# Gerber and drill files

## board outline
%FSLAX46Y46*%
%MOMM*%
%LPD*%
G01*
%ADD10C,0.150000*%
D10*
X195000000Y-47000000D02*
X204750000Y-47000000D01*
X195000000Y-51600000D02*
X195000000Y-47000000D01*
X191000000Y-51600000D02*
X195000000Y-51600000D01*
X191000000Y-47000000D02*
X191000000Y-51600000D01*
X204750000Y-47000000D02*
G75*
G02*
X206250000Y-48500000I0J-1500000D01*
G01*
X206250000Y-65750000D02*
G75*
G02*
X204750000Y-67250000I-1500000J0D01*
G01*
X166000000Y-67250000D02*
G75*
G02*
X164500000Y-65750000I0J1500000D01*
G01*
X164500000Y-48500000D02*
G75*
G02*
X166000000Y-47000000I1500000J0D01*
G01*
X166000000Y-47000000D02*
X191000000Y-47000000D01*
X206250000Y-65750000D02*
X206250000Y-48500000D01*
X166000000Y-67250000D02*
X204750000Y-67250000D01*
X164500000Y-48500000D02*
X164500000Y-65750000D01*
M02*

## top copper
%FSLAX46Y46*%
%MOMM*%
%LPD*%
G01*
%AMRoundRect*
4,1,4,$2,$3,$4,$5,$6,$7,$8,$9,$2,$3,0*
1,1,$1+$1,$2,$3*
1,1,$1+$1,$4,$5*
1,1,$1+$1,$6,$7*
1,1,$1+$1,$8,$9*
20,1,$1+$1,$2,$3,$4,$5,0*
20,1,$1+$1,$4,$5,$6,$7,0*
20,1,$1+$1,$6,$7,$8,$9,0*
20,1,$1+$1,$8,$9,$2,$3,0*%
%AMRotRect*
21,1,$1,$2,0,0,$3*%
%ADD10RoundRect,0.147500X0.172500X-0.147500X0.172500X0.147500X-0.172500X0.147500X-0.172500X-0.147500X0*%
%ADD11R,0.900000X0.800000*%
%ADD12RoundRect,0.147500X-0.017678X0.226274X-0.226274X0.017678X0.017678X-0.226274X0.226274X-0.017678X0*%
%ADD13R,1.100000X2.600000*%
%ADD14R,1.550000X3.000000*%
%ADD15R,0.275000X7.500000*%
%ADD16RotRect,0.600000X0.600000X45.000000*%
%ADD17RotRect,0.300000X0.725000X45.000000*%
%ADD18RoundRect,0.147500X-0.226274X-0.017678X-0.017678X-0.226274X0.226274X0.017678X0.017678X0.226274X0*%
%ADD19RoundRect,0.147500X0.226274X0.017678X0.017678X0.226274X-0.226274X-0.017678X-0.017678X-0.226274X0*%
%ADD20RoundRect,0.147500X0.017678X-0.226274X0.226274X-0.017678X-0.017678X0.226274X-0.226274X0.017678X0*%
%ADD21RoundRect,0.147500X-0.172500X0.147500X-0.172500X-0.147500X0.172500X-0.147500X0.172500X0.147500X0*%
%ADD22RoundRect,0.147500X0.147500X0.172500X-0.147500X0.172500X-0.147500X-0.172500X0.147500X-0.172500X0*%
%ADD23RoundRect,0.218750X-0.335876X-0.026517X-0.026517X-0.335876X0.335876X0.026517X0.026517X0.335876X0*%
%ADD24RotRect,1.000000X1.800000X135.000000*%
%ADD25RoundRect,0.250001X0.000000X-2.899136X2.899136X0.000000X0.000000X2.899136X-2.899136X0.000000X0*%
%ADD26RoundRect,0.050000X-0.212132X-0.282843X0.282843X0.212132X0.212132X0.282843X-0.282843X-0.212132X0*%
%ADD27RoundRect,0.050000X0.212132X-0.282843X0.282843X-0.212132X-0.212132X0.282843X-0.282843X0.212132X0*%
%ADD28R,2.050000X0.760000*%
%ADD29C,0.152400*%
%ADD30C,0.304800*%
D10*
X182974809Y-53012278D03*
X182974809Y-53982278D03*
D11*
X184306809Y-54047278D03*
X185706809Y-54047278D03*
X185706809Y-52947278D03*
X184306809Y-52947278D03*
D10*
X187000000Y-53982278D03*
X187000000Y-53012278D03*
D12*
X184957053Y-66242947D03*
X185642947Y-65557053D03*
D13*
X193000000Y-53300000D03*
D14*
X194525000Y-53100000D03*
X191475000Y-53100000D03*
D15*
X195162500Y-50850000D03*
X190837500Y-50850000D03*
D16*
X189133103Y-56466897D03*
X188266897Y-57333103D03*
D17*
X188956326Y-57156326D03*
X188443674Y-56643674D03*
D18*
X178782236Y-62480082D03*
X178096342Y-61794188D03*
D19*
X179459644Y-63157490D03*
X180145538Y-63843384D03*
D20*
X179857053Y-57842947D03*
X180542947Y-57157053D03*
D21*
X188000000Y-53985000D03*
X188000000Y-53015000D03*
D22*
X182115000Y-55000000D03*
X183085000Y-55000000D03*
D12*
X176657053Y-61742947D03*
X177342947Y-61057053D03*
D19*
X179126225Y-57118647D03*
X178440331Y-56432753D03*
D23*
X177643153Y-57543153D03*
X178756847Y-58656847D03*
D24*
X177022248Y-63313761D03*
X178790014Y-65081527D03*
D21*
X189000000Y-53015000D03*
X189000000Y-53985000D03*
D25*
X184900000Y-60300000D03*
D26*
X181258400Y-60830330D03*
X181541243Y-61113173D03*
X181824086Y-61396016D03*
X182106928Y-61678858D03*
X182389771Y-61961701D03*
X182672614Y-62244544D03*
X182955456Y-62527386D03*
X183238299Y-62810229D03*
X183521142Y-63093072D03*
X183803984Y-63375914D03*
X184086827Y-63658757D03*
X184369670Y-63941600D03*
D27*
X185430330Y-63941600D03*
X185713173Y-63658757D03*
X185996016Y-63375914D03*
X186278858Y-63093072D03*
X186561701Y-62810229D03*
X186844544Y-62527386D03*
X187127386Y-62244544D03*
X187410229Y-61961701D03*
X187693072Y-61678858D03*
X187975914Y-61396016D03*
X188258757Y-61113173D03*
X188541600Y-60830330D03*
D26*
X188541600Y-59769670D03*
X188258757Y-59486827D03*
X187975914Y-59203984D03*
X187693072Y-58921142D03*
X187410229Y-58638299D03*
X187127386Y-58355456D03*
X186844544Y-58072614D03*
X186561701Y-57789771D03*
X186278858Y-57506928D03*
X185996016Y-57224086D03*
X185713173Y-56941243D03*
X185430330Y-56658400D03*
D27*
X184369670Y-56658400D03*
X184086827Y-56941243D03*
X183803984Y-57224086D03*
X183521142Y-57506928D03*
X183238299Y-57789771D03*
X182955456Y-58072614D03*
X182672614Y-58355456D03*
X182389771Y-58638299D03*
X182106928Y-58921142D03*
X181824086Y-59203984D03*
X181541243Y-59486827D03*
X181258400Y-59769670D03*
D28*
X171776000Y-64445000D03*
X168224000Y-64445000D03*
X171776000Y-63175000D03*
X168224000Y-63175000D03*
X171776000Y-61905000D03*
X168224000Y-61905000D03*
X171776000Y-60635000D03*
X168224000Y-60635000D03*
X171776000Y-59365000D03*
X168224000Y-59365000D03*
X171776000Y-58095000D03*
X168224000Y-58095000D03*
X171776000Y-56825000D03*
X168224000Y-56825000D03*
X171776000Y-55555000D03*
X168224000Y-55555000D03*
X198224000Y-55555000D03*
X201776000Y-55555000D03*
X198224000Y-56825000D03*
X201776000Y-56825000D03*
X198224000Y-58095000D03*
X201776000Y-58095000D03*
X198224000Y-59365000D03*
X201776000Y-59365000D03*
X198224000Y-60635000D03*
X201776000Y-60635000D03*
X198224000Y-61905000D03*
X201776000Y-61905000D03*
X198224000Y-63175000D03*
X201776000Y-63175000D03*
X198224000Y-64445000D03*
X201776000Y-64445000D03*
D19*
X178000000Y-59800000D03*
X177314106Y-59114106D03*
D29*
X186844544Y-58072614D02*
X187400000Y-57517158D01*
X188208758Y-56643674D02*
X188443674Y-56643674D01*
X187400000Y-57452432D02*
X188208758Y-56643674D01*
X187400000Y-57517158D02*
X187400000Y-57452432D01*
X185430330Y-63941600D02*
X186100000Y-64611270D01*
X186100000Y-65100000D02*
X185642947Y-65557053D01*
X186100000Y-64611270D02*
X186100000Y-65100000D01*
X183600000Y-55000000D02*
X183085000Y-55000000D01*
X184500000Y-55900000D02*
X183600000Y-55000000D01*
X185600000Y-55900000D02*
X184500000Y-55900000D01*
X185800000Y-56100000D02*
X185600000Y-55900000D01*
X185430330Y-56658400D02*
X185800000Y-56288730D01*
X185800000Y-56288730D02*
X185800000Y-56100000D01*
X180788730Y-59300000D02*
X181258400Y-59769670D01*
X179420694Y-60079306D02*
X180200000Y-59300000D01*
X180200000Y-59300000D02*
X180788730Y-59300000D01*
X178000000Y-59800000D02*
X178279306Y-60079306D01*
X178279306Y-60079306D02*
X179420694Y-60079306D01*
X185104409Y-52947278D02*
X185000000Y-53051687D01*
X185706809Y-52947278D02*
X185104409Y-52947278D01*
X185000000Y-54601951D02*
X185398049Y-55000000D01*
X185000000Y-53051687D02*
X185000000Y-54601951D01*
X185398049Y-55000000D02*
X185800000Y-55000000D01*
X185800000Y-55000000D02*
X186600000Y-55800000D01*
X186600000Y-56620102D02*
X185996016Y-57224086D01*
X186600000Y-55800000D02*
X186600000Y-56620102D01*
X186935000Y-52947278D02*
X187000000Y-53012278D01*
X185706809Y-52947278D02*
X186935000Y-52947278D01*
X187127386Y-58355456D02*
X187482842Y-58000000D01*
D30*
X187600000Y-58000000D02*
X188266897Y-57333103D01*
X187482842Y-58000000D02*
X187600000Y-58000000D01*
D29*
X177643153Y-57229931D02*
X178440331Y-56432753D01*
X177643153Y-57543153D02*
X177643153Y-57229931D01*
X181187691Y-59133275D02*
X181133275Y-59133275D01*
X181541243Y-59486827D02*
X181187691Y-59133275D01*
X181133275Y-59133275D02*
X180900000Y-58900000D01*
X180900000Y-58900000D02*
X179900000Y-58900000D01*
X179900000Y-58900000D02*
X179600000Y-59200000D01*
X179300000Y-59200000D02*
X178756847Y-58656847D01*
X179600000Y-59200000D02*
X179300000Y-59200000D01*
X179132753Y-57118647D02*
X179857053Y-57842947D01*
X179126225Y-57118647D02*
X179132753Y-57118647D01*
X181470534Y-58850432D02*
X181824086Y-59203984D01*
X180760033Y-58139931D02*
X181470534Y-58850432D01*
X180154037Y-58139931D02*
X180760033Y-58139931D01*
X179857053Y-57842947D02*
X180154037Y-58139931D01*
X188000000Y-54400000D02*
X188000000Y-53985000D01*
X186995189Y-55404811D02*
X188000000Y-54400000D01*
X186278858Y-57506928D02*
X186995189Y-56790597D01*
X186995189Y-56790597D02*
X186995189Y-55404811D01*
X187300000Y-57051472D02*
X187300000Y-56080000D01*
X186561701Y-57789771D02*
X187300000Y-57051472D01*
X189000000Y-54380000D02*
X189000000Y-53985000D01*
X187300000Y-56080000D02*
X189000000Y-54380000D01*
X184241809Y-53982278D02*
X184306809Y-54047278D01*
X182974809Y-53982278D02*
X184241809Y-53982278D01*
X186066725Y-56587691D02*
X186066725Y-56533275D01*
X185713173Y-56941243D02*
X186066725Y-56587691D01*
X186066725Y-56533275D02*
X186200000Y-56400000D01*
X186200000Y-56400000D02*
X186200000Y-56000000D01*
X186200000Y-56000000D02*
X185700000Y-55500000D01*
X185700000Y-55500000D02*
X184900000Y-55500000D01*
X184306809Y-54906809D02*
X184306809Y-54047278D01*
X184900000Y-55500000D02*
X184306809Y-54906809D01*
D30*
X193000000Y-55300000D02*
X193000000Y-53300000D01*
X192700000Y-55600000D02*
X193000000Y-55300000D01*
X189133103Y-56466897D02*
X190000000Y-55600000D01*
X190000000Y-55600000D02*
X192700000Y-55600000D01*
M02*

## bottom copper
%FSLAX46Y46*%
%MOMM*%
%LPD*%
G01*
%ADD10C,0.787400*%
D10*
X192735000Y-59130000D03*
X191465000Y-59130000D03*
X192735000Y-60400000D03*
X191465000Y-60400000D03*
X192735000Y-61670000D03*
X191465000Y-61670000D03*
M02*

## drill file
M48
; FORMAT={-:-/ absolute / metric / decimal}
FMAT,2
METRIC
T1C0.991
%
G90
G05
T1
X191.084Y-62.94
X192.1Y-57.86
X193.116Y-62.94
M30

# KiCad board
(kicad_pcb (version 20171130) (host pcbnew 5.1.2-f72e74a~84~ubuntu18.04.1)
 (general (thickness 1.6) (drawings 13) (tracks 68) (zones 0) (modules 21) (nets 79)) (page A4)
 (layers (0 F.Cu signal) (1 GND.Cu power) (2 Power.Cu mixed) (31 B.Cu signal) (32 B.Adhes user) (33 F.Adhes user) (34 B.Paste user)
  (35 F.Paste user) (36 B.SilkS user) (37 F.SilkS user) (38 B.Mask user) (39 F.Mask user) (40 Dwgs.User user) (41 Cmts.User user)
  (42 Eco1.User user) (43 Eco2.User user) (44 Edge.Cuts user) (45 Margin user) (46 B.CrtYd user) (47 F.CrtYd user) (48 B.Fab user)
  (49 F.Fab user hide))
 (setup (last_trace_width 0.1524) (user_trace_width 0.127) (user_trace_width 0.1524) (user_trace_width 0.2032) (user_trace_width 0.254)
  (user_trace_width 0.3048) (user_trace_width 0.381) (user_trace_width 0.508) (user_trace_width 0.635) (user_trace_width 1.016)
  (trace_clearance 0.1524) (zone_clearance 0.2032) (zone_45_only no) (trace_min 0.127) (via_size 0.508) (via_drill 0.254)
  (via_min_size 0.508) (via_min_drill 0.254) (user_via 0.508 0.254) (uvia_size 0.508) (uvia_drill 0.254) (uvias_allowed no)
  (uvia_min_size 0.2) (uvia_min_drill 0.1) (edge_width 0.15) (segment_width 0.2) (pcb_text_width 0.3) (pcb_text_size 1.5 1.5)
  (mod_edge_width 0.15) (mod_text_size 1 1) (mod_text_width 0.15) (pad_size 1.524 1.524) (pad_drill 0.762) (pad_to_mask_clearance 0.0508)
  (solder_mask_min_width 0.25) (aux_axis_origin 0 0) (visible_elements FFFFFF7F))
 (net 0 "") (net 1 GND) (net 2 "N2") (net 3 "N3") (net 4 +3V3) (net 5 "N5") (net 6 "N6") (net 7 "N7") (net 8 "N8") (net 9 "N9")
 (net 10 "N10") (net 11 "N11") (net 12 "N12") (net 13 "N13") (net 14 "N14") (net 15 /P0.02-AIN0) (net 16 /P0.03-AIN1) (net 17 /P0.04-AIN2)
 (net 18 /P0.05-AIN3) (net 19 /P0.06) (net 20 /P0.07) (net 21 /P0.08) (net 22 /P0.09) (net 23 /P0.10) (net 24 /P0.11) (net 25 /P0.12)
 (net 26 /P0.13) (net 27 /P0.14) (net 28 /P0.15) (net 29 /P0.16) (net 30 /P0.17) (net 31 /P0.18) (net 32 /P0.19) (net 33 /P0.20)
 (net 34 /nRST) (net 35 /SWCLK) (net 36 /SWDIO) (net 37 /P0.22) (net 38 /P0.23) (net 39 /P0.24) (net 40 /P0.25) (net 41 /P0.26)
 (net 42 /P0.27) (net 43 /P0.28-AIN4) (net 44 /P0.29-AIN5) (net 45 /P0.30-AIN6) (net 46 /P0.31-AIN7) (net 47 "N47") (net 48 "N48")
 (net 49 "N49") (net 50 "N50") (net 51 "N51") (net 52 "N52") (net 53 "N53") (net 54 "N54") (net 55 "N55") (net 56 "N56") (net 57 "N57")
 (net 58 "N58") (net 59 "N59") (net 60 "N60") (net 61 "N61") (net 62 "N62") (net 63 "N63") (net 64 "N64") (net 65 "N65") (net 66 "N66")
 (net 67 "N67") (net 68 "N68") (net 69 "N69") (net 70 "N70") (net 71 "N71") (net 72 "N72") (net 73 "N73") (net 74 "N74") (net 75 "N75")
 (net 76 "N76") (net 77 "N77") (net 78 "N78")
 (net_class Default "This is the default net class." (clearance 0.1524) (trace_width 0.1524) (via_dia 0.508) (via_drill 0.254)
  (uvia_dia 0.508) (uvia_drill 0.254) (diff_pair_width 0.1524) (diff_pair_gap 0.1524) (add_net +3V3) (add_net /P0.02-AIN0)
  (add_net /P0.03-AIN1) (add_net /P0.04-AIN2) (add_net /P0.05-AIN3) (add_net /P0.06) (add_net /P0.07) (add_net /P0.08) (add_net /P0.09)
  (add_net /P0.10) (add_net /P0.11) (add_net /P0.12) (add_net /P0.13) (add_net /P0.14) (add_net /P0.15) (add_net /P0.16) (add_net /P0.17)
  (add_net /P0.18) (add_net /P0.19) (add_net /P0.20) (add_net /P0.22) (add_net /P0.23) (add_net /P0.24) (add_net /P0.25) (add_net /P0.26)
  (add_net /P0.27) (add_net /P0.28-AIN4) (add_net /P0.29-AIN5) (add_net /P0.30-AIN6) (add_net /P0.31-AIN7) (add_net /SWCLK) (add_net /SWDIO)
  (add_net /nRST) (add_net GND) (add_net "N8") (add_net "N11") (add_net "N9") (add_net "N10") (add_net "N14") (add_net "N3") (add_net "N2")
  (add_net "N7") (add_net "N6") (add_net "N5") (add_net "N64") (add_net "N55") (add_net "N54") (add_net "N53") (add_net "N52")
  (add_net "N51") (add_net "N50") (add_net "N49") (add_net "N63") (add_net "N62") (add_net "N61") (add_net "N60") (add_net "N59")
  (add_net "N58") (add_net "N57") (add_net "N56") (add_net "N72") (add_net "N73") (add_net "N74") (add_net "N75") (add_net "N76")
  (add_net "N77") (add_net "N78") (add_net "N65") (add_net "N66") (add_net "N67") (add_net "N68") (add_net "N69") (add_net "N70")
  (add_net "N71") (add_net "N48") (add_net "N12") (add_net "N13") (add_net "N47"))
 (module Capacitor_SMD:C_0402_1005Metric (layer F.Cu) (at 182.974809 53.497278 90)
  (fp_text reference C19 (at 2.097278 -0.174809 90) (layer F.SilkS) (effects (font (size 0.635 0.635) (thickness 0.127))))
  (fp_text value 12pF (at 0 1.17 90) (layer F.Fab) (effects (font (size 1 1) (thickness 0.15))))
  (pad 2 smd roundrect (at 0.485 0 90) (size 0.59 0.64) (layers F.Cu F.Paste F.Mask) (roundrect_rratio 0.25) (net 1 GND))
  (pad 1 smd roundrect (at -0.485 0 90) (size 0.59 0.64) (layers F.Cu F.Paste F.Mask) (roundrect_rratio 0.25) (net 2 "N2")))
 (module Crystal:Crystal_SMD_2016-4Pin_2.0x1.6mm (layer F.Cu) (at 185.006809 53.497278)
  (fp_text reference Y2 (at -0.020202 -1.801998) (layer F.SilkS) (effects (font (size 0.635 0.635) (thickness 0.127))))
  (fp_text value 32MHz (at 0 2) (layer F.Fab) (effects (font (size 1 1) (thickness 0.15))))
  (pad 1 smd rect (at -0.7 0.55) (size 0.9 0.8) (layers F.Cu F.Paste F.Mask) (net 2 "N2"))
  (pad 2 smd rect (at 0.7 0.55) (size 0.9 0.8) (layers F.Cu F.Paste F.Mask) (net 1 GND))
  (pad 3 smd rect (at 0.7 -0.55) (size 0.9 0.8) (layers F.Cu F.Paste F.Mask) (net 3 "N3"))
  (pad 4 smd rect (at -0.7 -0.55) (size 0.9 0.8) (layers F.Cu F.Paste F.Mask) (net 1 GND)))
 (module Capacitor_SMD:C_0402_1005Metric (layer F.Cu) (at 187 53.497278 90)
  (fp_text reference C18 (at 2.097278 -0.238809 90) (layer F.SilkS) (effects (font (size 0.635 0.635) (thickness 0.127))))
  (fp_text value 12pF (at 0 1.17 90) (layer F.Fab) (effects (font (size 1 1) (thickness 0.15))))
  (pad 1 smd roundrect (at -0.485 0 90) (size 0.59 0.64) (layers F.Cu F.Paste F.Mask) (roundrect_rratio 0.25) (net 1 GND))
  (pad 2 smd roundrect (at 0.485 0 90) (size 0.59 0.64) (layers F.Cu F.Paste F.Mask) (roundrect_rratio 0.25) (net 3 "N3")))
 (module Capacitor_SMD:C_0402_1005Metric (layer F.Cu) (at 185.3 65.9 225)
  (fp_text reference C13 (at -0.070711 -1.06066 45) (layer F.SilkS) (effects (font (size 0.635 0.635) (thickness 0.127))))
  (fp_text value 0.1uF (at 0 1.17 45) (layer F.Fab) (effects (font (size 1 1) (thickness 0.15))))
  (pad 2 smd roundrect (at 0.485 0 225) (size 0.59 0.64) (layers F.Cu F.Paste F.Mask) (roundrect_rratio 0.25) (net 1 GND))
  (pad 1 smd roundrect (at -0.485 0 225) (size 0.59 0.64) (layers F.Cu F.Paste F.Mask) (roundrect_rratio 0.25) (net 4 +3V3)))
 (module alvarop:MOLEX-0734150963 (layer F.Cu) (at 193 54.6 270)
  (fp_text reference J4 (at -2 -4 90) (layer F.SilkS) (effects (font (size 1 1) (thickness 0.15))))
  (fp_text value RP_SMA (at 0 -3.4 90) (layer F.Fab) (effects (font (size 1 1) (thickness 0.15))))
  (pad 1 smd rect (at -1.3 0 270) (size 2.6 1.1) (layers F.Cu F.Paste F.Mask) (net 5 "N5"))
  (pad 2 smd rect (at -1.5 -1.525 270) (size 3 1.55) (layers F.Cu F.Paste F.Mask) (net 1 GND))
  (pad 2 smd rect (at -1.5 1.525 270) (size 3 1.55) (layers F.Cu F.Paste F.Mask) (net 1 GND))
  (pad 2 smd rect (at -3.75 -2.1625 270) (size 7.5 0.275) (layers F.Cu F.Paste F.Mask) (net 1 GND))
  (pad 2 smd rect (at -3.75 2.1625 270) (size 7.5 0.275) (layers F.Cu F.Paste F.Mask) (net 1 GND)))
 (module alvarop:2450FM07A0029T (layer F.Cu) (at 188.7 56.9 45)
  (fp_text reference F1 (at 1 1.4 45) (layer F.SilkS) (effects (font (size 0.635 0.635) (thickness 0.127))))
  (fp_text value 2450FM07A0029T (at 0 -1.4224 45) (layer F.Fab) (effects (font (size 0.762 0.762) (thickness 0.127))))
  (pad 3 smd rect (at 0.6125 0 45) (size 0.6 0.6) (layers F.Cu F.Paste F.Mask) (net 5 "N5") (solder_paste_margin -0.0508))
  (pad 1 smd rect (at -0.6125 0 45) (size 0.6 0.6) (layers F.Cu F.Paste F.Mask) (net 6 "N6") (solder_paste_margin -0.0508))
  (pad 2 smd rect (at 0 0.3625 45) (size 0.3 0.725) (layers F.Cu F.Paste F.Mask) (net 1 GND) (solder_paste_margin -0.0508))
  (pad 4 smd rect (at 0 -0.3625 45) (size 0.3 0.725) (layers F.Cu F.Paste F.Mask) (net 1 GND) (solder_paste_margin -0.0508)))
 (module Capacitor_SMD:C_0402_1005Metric (layer F.Cu) (at 178.439289 62.137135 315)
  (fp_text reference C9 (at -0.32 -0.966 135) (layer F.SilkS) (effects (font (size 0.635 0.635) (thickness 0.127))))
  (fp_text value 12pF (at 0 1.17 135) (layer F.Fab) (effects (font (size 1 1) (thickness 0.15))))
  (pad 2 smd roundrect (at 0.485 0 315) (size 0.59 0.64) (layers F.Cu F.Paste F.Mask) (roundrect_rratio 0.25) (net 1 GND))
  (pad 1 smd roundrect (at -0.485 0 315) (size 0.59 0.64) (layers F.Cu F.Paste F.Mask) (roundrect_rratio 0.25) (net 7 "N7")))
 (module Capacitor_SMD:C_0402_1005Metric (layer F.Cu) (at 179.802591 63.500437 135)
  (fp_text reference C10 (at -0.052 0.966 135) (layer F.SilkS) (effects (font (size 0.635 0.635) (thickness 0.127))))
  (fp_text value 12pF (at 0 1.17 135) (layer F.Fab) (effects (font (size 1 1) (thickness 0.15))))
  (pad 2 smd roundrect (at 0.485 0 135) (size 0.59 0.64) (layers F.Cu F.Paste F.Mask) (roundrect_rratio 0.25) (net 1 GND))
  (pad 1 smd roundrect (at -0.485 0 135) (size 0.59 0.64) (layers F.Cu F.Paste F.Mask) (roundrect_rratio 0.25) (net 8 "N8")))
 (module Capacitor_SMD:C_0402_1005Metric (layer F.Cu) (at 180.2 57.5 45)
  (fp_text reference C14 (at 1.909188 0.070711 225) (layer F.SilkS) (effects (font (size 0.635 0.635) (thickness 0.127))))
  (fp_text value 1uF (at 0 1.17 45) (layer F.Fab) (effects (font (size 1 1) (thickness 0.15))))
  (pad 1 smd roundrect (at -0.485 0 45) (size 0.59 0.64) (layers F.Cu F.Paste F.Mask) (roundrect_rratio 0.25) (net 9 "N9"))
  (pad 2 smd roundrect (at 0.485 0 45) (size 0.59 0.64) (layers F.Cu F.Paste F.Mask) (roundrect_rratio 0.25) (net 1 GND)))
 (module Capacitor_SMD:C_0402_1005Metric (layer F.Cu) (at 188 53.5 270)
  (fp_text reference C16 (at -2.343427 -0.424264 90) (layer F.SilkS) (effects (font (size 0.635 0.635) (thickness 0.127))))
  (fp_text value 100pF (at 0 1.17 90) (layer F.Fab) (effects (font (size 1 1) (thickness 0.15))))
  (pad 2 smd roundrect (at 0.485 0 270) (size 0.59 0.64) (layers F.Cu F.Paste F.Mask) (roundrect_rratio 0.25) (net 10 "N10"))
  (pad 1 smd roundrect (at -0.485 0 270) (size 0.59 0.64) (layers F.Cu F.Paste F.Mask) (roundrect_rratio 0.25) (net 1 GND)))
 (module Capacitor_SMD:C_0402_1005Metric (layer F.Cu) (at 182.6 55 180)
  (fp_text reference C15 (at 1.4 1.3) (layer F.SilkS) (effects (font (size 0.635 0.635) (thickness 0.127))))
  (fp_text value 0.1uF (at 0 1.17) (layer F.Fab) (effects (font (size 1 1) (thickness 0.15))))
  (pad 2 smd roundrect (at 0.485 0 180) (size 0.59 0.64) (layers F.Cu F.Paste F.Mask) (roundrect_rratio 0.25) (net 1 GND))
  (pad 1 smd roundrect (at -0.485 0 180) (size 0.59 0.64) (layers F.Cu F.Paste F.Mask) (roundrect_rratio 0.25) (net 4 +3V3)))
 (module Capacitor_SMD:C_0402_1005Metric (layer F.Cu) (at 177 61.4 225)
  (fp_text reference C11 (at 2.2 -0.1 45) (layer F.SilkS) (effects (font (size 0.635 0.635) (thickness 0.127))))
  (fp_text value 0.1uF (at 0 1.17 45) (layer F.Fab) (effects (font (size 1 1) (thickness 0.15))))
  (pad 2 smd roundrect (at 0.485 0 225) (size 0.59 0.64) (layers F.Cu F.Paste F.Mask) (roundrect_rratio 0.25) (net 1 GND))
  (pad 1 smd roundrect (at -0.485 0 225) (size 0.59 0.64) (layers F.Cu F.Paste F.Mask) (roundrect_rratio 0.25) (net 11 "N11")))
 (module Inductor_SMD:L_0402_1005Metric (layer F.Cu) (at 178.783278 56.7757 135)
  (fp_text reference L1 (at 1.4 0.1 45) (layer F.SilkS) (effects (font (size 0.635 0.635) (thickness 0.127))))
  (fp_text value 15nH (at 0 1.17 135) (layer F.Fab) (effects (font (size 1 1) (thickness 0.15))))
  (pad 1 smd roundrect (at -0.485 0 135) (size 0.59 0.64) (layers F.Cu F.Paste F.Mask) (roundrect_rratio 0.25) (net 9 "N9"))
  (pad 2 smd roundrect (at 0.485 0 135) (size 0.59 0.64) (layers F.Cu F.Paste F.Mask) (roundrect_rratio 0.25) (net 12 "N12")))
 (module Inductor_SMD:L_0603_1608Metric (layer F.Cu) (at 178.2 58.1 315)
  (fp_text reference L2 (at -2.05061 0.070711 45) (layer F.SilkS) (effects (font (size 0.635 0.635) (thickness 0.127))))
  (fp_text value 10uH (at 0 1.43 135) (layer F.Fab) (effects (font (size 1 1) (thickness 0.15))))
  (pad 1 smd roundrect (at -0.7875 0 315) (size 0.875 0.95) (layers F.Cu F.Paste F.Mask) (roundrect_rratio 0.25) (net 12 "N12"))
  (pad 2 smd roundrect (at 0.7875 0 315) (size 0.875 0.95) (layers F.Cu F.Paste F.Mask) (roundrect_rratio 0.25) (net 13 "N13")))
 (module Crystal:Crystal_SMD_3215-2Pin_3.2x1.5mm (layer F.Cu) (at 177.906131 64.197644 135)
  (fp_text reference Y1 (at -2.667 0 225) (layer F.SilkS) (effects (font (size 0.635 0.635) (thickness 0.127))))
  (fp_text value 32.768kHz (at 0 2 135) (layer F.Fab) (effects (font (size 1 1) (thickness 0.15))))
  (pad 1 smd rect (at 1.25 0 135) (size 1 1.8) (layers F.Cu F.Paste F.Mask) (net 7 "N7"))
  (pad 2 smd rect (at -1.25 0 135) (size 1 1.8) (layers F.Cu F.Paste F.Mask) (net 8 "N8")))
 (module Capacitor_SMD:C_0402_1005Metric (layer F.Cu) (at 189 53.5 270)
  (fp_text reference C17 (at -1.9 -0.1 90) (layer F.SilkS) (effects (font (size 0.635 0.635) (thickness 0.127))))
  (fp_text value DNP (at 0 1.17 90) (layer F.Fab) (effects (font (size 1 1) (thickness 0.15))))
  (pad 1 smd roundrect (at -0.485 0 270) (size 0.59 0.64) (layers F.Cu F.Paste F.Mask) (roundrect_rratio 0.25) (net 1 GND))
  (pad 2 smd roundrect (at 0.485 0 270) (size 0.59 0.64) (layers F.Cu F.Paste F.Mask) (roundrect_rratio 0.25) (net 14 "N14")))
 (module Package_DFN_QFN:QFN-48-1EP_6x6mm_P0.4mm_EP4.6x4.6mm (layer F.Cu) (at 184.9 60.3 45)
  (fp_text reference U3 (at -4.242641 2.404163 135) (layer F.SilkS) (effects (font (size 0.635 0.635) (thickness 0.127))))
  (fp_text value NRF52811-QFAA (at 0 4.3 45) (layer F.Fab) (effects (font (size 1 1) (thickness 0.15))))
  (pad 49 smd roundrect (at 0 0 45) (size 4.6 4.6) (layers F.Cu F.Mask) (roundrect_rratio 0.054348) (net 1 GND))
  (pad "" smd roundrect (at -1.53 -1.53 45) (size 1.24 1.24) (layers F.Paste) (roundrect_rratio 0.201613))
  (pad "" smd roundrect (at -1.53 0 45) (size 1.24 1.24) (layers F.Paste) (roundrect_rratio 0.201613))
  (pad "" smd roundrect (at -1.53 1.53 45) (size 1.24 1.24) (layers F.Paste) (roundrect_rratio 0.201613))
  (pad "" smd roundrect (at 0 -1.53 45) (size 1.24 1.24) (layers F.Paste) (roundrect_rratio 0.201613))
  (pad "" smd roundrect (at 0 0 45) (size 1.24 1.24) (layers F.Paste) (roundrect_rratio 0.201613))
  (pad "" smd roundrect (at 0 1.53 45) (size 1.24 1.24) (layers F.Paste) (roundrect_rratio 0.201613))
  (pad "" smd roundrect (at 1.53 -1.53 45) (size 1.24 1.24) (layers F.Paste) (roundrect_rratio 0.201613))
  (pad "" smd roundrect (at 1.53 0 45) (size 1.24 1.24) (layers F.Paste) (roundrect_rratio 0.201613))
  (pad "" smd roundrect (at 1.53 1.53 45) (size 1.24 1.24) (layers F.Paste) (roundrect_rratio 0.201613))
  (pad 1 smd roundrect (at -2.95 -2.2 45) (size 0.8 0.2) (layers F.Cu F.Paste F.Mask) (roundrect_rratio 0.25) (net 11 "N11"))
  (pad 2 smd roundrect (at -2.95 -1.8 45) (size 0.8 0.2) (layers F.Cu F.Paste F.Mask) (roundrect_rratio 0.25) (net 7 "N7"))
  (pad 3 smd roundrect (at -2.95 -1.4 45) (size 0.8 0.2) (layers F.Cu F.Paste F.Mask) (roundrect_rratio 0.25) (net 8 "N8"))
  (pad 4 smd roundrect (at -2.95 -1 45) (size 0.8 0.2) (layers F.Cu F.Paste F.Mask) (roundrect_rratio 0.25) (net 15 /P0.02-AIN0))
  (pad 5 smd roundrect (at -2.95 -0.6 45) (size 0.8 0.2) (layers F.Cu F.Paste F.Mask) (roundrect_rratio 0.25) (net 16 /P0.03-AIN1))
  (pad 6 smd roundrect (at -2.95 -0.2 45) (size 0.8 0.2) (layers F.Cu F.Paste F.Mask) (roundrect_rratio 0.25) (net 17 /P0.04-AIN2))
  (pad 7 smd roundrect (at -2.95 0.2 45) (size 0.8 0.2) (layers F.Cu F.Paste F.Mask) (roundrect_rratio 0.25) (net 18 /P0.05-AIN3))
  (pad 8 smd roundrect (at -2.95 0.6 45) (size 0.8 0.2) (layers F.Cu F.Paste F.Mask) (roundrect_rratio 0.25) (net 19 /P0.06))
  (pad 9 smd roundrect (at -2.95 1 45) (size 0.8 0.2) (layers F.Cu F.Paste F.Mask) (roundrect_rratio 0.25) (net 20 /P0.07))
  (pad 10 smd roundrect (at -2.95 1.4 45) (size 0.8 0.2) (layers F.Cu F.Paste F.Mask) (roundrect_rratio 0.25) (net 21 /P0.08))
  (pad 11 smd roundrect (at -2.95 1.8 45) (size 0.8 0.2) (layers F.Cu F.Paste F.Mask) (roundrect_rratio 0.25) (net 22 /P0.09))
  (pad 12 smd roundrect (at -2.95 2.2 45) (size 0.8 0.2) (layers F.Cu F.Paste F.Mask) (roundrect_rratio 0.25) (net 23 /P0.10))
  (pad 13 smd roundrect (at -2.2 2.95 45) (size 0.2 0.8) (layers F.Cu F.Paste F.Mask) (roundrect_rratio 0.25) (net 4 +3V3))
  (pad 14 smd roundrect (at -1.8 2.95 45) (size 0.2 0.8) (layers F.Cu F.Paste F.Mask) (roundrect_rratio 0.25) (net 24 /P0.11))
  (pad 15 smd roundrect (at -1.4 2.95 45) (size 0.2 0.8) (layers F.Cu F.Paste F.Mask) (roundrect_rratio 0.25) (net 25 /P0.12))
  (pad 16 smd roundrect (at -1 2.95 45) (size 0.2 0.8) (layers F.Cu F.Paste F.Mask) (roundrect_rratio 0.25) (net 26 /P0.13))
  (pad 17 smd roundrect (at -0.6 2.95 45) (size 0.2 0.8) (layers F.Cu F.Paste F.Mask) (roundrect_rratio 0.25) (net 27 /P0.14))
  (pad 18 smd roundrect (at -0.2 2.95 45) (size 0.2 0.8) (layers F.Cu F.Paste F.Mask) (roundrect_rratio 0.25) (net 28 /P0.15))
  (pad 19 smd roundrect (at 0.2 2.95 45) (size 0.2 0.8) (layers F.Cu F.Paste F.Mask) (roundrect_rratio 0.25) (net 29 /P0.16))
  (pad 20 smd roundrect (at 0.6 2.95 45) (size 0.2 0.8) (layers F.Cu F.Paste F.Mask) (roundrect_rratio 0.25) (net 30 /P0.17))
  (pad 21 smd roundrect (at 1 2.95 45) (size 0.2 0.8) (layers F.Cu F.Paste F.Mask) (roundrect_rratio 0.25) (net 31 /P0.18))
  (pad 22 smd roundrect (at 1.4 2.95 45) (size 0.2 0.8) (layers F.Cu F.Paste F.Mask) (roundrect_rratio 0.25) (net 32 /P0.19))
  (pad 23 smd roundrect (at 1.8 2.95 45) (size 0.2 0.8) (layers F.Cu F.Paste F.Mask) (roundrect_rratio 0.25) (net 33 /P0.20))
  (pad 24 smd roundrect (at 2.2 2.95 45) (size 0.2 0.8) (layers F.Cu F.Paste F.Mask) (roundrect_rratio 0.25) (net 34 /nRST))
  (pad 25 smd roundrect (at 2.95 2.2 45) (size 0.8 0.2) (layers F.Cu F.Paste F.Mask) (roundrect_rratio 0.25) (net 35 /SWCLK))
  (pad 26 smd roundrect (at 2.95 1.8 45) (size 0.8 0.2) (layers F.Cu F.Paste F.Mask) (roundrect_rratio 0.25) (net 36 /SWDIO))
  (pad 27 smd roundrect (at 2.95 1.4 45) (size 0.8 0.2) (layers F.Cu F.Paste F.Mask) (roundrect_rratio 0.25) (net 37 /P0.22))
  (pad 28 smd roundrect (at 2.95 1 45) (size 0.8 0.2) (layers F.Cu F.Paste F.Mask) (roundrect_rratio 0.25) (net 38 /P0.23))
  (pad 29 smd roundrect (at 2.95 0.6 45) (size 0.8 0.2) (layers F.Cu F.Paste F.Mask) (roundrect_rratio 0.25) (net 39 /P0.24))
  (pad 30 smd roundrect (at 2.95 0.2 45) (size 0.8 0.2) (layers F.Cu F.Paste F.Mask) (roundrect_rratio 0.25) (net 6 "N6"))
  (pad 31 smd roundrect (at 2.95 -0.2 45) (size 0.8 0.2) (layers F.Cu F.Paste F.Mask) (roundrect_rratio 0.25) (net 1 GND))
  (pad 32 smd roundrect (at 2.95 -0.6 45) (size 0.8 0.2) (layers F.Cu F.Paste F.Mask) (roundrect_rratio 0.25) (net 14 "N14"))
  (pad 33 smd roundrect (at 2.95 -1 45) (size 0.8 0.2) (layers F.Cu F.Paste F.Mask) (roundrect_rratio 0.25) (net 10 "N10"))
  (pad 34 smd roundrect (at 2.95 -1.4 45) (size 0.8 0.2) (layers F.Cu F.Paste F.Mask) (roundrect_rratio 0.25) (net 3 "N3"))
  (pad 35 smd roundrect (at 2.95 -1.8 45) (size 0.8 0.2) (layers F.Cu F.Paste F.Mask) (roundrect_rratio 0.25) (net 2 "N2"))
  (pad 36 smd roundrect (at 2.95 -2.2 45) (size 0.8 0.2) (layers F.Cu F.Paste F.Mask) (roundrect_rratio 0.25) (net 4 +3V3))
  (pad 37 smd roundrect (at 2.2 -2.95 45) (size 0.2 0.8) (layers F.Cu F.Paste F.Mask) (roundrect_rratio 0.25) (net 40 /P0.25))
  (pad 38 smd roundrect (at 1.8 -2.95 45) (size 0.2 0.8) (layers F.Cu F.Paste F.Mask) (roundrect_rratio 0.25) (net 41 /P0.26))
  (pad 39 smd roundrect (at 1.4 -2.95 45) (size 0.2 0.8) (layers F.Cu F.Paste F.Mask) (roundrect_rratio 0.25) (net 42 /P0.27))
  (pad 40 smd roundrect (at 1 -2.95 45) (size 0.2 0.8) (layers F.Cu F.Paste F.Mask) (roundrect_rratio 0.25) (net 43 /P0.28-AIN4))
  (pad 41 smd roundrect (at 0.6 -2.95 45) (size 0.2 0.8) (layers F.Cu F.Paste F.Mask) (roundrect_rratio 0.25) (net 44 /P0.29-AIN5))
  (pad 42 smd roundrect (at 0.2 -2.95 45) (size 0.2 0.8) (layers F.Cu F.Paste F.Mask) (roundrect_rratio 0.25) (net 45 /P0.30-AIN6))
  (pad 43 smd roundrect (at -0.2 -2.95 45) (size 0.2 0.8) (layers F.Cu F.Paste F.Mask) (roundrect_rratio 0.25) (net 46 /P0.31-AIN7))
  (pad 44 smd roundrect (at -0.6 -2.95 45) (size 0.2 0.8) (layers F.Cu F.Paste F.Mask) (roundrect_rratio 0.25) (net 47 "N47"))
  (pad 45 smd roundrect (at -1 -2.95 45) (size 0.2 0.8) (layers F.Cu F.Paste F.Mask) (roundrect_rratio 0.25) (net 1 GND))
  (pad 46 smd roundrect (at -1.4 -2.95 45) (size 0.2 0.8) (layers F.Cu F.Paste F.Mask) (roundrect_rratio 0.25) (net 9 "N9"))
  (pad 47 smd roundrect (at -1.8 -2.95 45) (size 0.2 0.8) (layers F.Cu F.Paste F.Mask) (roundrect_rratio 0.25) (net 13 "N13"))
  (pad 48 smd roundrect (at -2.2 -2.95 45) (size 0.2 0.8) (layers F.Cu F.Paste F.Mask) (roundrect_rratio 0.25) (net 4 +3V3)))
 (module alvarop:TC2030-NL (layer B.Cu) (at 192.1 60.4 270)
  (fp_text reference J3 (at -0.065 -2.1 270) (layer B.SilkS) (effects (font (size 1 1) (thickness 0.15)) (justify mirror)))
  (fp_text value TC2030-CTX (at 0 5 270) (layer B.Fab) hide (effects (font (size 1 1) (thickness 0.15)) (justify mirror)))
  (pad 1 smd circle (at -1.27 -0.635 270) (size 0.7874 0.7874) (layers B.Cu B.Mask) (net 4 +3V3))
  (pad 2 smd circle (at -1.27 0.635 270) (size 0.7874 0.7874) (layers B.Cu B.Mask) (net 36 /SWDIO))
  (pad 3 smd circle (at 0 -0.635 270) (size 0.7874 0.7874) (layers B.Cu B.Mask) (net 34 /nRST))
  (pad 4 smd circle (at 0 0.635 270) (size 0.7874 0.7874) (layers B.Cu B.Mask) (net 35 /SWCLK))
  (pad 5 smd circle (at 1.27 -0.635 270) (size 0.7874 0.7874) (layers B.Cu B.Mask) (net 1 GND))
  (pad 6 smd circle (at 1.27 0.635 270) (size 0.7874 0.7874) (layers B.Cu B.Mask) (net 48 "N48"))
  (pad "" np_thru_hole circle (at 2.54 -1.016 270) (size 0.9906 0.9906) (drill 0.9906) (layers *.Cu *.Mask))
  (pad "" np_thru_hole circle (at 2.54 1.016 270) (size 0.9906 0.9906) (drill 0.9906) (layers *.Cu *.Mask))
  (pad "" np_thru_hole circle (at -2.54 0 270) (size 0.9906 0.9906) (drill 0.9906) (layers *.Cu *.Mask)))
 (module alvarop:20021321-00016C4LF (layer F.Cu) (at 170 60 270)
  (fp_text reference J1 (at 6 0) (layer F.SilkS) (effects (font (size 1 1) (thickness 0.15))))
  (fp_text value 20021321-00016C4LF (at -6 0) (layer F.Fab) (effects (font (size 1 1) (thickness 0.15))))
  (pad 16 smd rect (at 4.445 -1.776 270) (size 0.76 2.05) (layers F.Cu F.Paste F.Mask) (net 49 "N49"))
  (pad 15 smd rect (at 4.445 1.776 270) (size 0.76 2.05) (layers F.Cu F.Paste F.Mask) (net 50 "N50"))
  (pad 14 smd rect (at 3.175 -1.776 270) (size 0.76 2.05) (layers F.Cu F.Paste F.Mask) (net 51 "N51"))
  (pad 13 smd rect (at 3.175 1.776 270) (size 0.76 2.05) (layers F.Cu F.Paste F.Mask) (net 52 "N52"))
  (pad 12 smd rect (at 1.905 -1.776 270) (size 0.76 2.05) (layers F.Cu F.Paste F.Mask) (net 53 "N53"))
  (pad 11 smd rect (at 1.905 1.776 270) (size 0.76 2.05) (layers F.Cu F.Paste F.Mask) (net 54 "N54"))
  (pad 10 smd rect (at 0.635 -1.776 270) (size 0.76 2.05) (layers F.Cu F.Paste F.Mask) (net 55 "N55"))
  (pad 9 smd rect (at 0.635 1.776 270) (size 0.76 2.05) (layers F.Cu F.Paste F.Mask) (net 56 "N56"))
  (pad 8 smd rect (at -0.635 -1.776 270) (size 0.76 2.05) (layers F.Cu F.Paste F.Mask) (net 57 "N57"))
  (pad 7 smd rect (at -0.635 1.776 270) (size 0.76 2.05) (layers F.Cu F.Paste F.Mask) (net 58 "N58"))
  (pad 6 smd rect (at -1.905 -1.776 270) (size 0.76 2.05) (layers F.Cu F.Paste F.Mask) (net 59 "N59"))
  (pad 5 smd rect (at -1.905 1.776 270) (size 0.76 2.05) (layers F.Cu F.Paste F.Mask) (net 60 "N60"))
  (pad 4 smd rect (at -3.175 -1.776 270) (size 0.76 2.05) (layers F.Cu F.Paste F.Mask) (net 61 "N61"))
  (pad 3 smd rect (at -3.175 1.776 270) (size 0.76 2.05) (layers F.Cu F.Paste F.Mask) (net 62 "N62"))
  (pad 2 smd rect (at -4.445 -1.776 270) (size 0.76 2.05) (layers F.Cu F.Paste F.Mask) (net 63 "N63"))
  (pad 1 smd rect (at -4.445 1.776 270) (size 0.76 2.05) (layers F.Cu F.Paste F.Mask) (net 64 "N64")))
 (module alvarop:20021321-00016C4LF (layer F.Cu) (at 200 60 270)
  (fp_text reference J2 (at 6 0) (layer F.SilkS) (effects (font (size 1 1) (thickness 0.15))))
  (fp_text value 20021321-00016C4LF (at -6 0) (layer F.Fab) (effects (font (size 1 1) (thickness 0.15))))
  (pad 1 smd rect (at -4.445 1.776 270) (size 0.76 2.05) (layers F.Cu F.Paste F.Mask) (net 4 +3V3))
  (pad 2 smd rect (at -4.445 -1.776 270) (size 0.76 2.05) (layers F.Cu F.Paste F.Mask) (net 1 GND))
  (pad 3 smd rect (at -3.175 1.776 270) (size 0.76 2.05) (layers F.Cu F.Paste F.Mask) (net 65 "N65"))
  (pad 4 smd rect (at -3.175 -1.776 270) (size 0.76 2.05) (layers F.Cu F.Paste F.Mask) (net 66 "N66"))
  (pad 5 smd rect (at -1.905 1.776 270) (size 0.76 2.05) (layers F.Cu F.Paste F.Mask) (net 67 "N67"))
  (pad 6 smd rect (at -1.905 -1.776 270) (size 0.76 2.05) (layers F.Cu F.Paste F.Mask) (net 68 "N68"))
  (pad 7 smd rect (at -0.635 1.776 270) (size 0.76 2.05) (layers F.Cu F.Paste F.Mask) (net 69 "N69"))
  (pad 8 smd rect (at -0.635 -1.776 270) (size 0.76 2.05) (layers F.Cu F.Paste F.Mask) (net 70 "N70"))
  (pad 9 smd rect (at 0.635 1.776 270) (size 0.76 2.05) (layers F.Cu F.Paste F.Mask) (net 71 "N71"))
  (pad 10 smd rect (at 0.635 -1.776 270) (size 0.76 2.05) (layers F.Cu F.Paste F.Mask) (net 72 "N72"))
  (pad 11 smd rect (at 1.905 1.776 270) (size 0.76 2.05) (layers F.Cu F.Paste F.Mask) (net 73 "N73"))
  (pad 12 smd rect (at 1.905 -1.776 270) (size 0.76 2.05) (layers F.Cu F.Paste F.Mask) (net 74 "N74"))
  (pad 13 smd rect (at 3.175 1.776 270) (size 0.76 2.05) (layers F.Cu F.Paste F.Mask) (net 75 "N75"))
  (pad 14 smd rect (at 3.175 -1.776 270) (size 0.76 2.05) (layers F.Cu F.Paste F.Mask) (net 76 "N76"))
  (pad 15 smd rect (at 4.445 1.776 270) (size 0.76 2.05) (layers F.Cu F.Paste F.Mask) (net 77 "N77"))
  (pad 16 smd rect (at 4.445 -1.776 270) (size 0.76 2.05) (layers F.Cu F.Paste F.Mask) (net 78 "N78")))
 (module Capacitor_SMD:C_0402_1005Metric (layer F.Cu) (at 177.657053 59.457053 135)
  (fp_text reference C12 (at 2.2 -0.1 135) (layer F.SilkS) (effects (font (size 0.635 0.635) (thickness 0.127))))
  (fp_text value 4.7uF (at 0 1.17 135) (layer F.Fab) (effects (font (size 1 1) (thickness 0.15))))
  (pad 1 smd roundrect (at -0.485 0 135) (size 0.59 0.64) (layers F.Cu F.Paste F.Mask) (roundrect_rratio 0.25) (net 4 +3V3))
  (pad 2 smd roundrect (at 0.485 0 135) (size 0.59 0.64) (layers F.Cu F.Paste F.Mask) (roundrect_rratio 0.25) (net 1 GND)))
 (gr_line (start 195 47) (end 204.75 47) (layer Edge.Cuts) (width 0.15))
 (gr_line (start 195 51.6) (end 195 47) (layer Edge.Cuts) (width 0.15))
 (gr_line (start 191 51.6) (end 195 51.6) (layer Edge.Cuts) (width 0.15))
 (gr_line (start 191 47) (end 191 51.6) (layer Edge.Cuts) (width 0.15))
 (gr_arc (start 204.75 48.5) (end 206.25 48.5) (angle -90) (layer Edge.Cuts) (width 0.15))
 (gr_arc (start 204.75 65.75) (end 204.75 67.25) (angle -90) (layer Edge.Cuts) (width 0.15))
 (gr_arc (start 166 65.75) (end 164.5 65.75) (angle -90) (layer Edge.Cuts) (width 0.15))
 (gr_arc (start 166 48.5) (end 166 47) (angle -90) (layer Edge.Cuts) (width 0.15))
 (gr_line (start 166 47) (end 191 47) (layer Edge.Cuts) (width 0.15))
 (gr_line (start 206.25 65.75) (end 206.25 48.5) (layer Edge.Cuts) (width 0.15))
 (gr_line (start 166 67.25) (end 204.75 67.25) (layer Edge.Cuts) (width 0.15))
 (gr_line (start 164.5 48.5) (end 164.5 65.75) (layer Edge.Cuts) (width 0.15))
 (segment (start 186.844544 58.072614) (end 187.4 57.517158) (width 0.1524) (layer F.Cu) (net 1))
 (segment (start 188.208758 56.643674) (end 188.443674 56.643674) (width 0.1524) (layer F.Cu) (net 1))
 (segment (start 187.4 57.452432) (end 188.208758 56.643674) (width 0.1524) (layer F.Cu) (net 1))
 (segment (start 187.4 57.517158) (end 187.4 57.452432) (width 0.1524) (layer F.Cu) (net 1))
 (segment (start 185.43033 63.9416) (end 186.1 64.61127) (width 0.1524) (layer F.Cu) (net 4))
 (segment (start 186.1 65.1) (end 185.642947 65.557053) (width 0.1524) (layer F.Cu) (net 4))
 (segment (start 186.1 64.61127) (end 186.1 65.1) (width 0.1524) (layer F.Cu) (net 4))
 (segment (start 183.6 55) (end 183.085 55) (width 0.1524) (layer F.Cu) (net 4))
 (segment (start 184.5 55.9) (end 183.6 55) (width 0.1524) (layer F.Cu) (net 4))
 (segment (start 185.6 55.9) (end 184.5 55.9) (width 0.1524) (layer F.Cu) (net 4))
 (segment (start 185.8 56.1) (end 185.6 55.9) (width 0.1524) (layer F.Cu) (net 4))
 (segment (start 185.43033 56.6584) (end 185.8 56.28873) (width 0.1524) (layer F.Cu) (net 4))
 (segment (start 185.8 56.28873) (end 185.8 56.1) (width 0.1524) (layer F.Cu) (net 4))
 (segment (start 180.78873 59.3) (end 181.2584 59.76967) (width 0.1524) (layer F.Cu) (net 4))
 (segment (start 179.420694 60.079306) (end 180.2 59.3) (width 0.1524) (layer F.Cu) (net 4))
 (segment (start 180.2 59.3) (end 180.78873 59.3) (width 0.1524) (layer F.Cu) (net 4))
 (segment (start 178 59.8) (end 178.279306 60.079306) (width 0.1524) (layer F.Cu) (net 4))
 (segment (start 178.279306 60.079306) (end 179.420694 60.079306) (width 0.1524) (layer F.Cu) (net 4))
 (segment (start 185.104409 52.947278) (end 185 53.051687) (width 0.1524) (layer F.Cu) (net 3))
 (segment (start 185.706809 52.947278) (end 185.104409 52.947278) (width 0.1524) (layer F.Cu) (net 3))
 (segment (start 185 54.601951) (end 185.398049 55) (width 0.1524) (layer F.Cu) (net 3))
 (segment (start 185 53.051687) (end 185 54.601951) (width 0.1524) (layer F.Cu) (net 3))
 (segment (start 185.398049 55) (end 185.8 55) (width 0.1524) (layer F.Cu) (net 3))
 (segment (start 185.8 55) (end 186.6 55.8) (width 0.1524) (layer F.Cu) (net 3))
 (segment (start 186.6 56.620102) (end 185.996016 57.224086) (width 0.1524) (layer F.Cu) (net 3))
 (segment (start 186.6 55.8) (end 186.6 56.620102) (width 0.1524) (layer F.Cu) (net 3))
 (segment (start 186.935 52.947278) (end 187 53.012278) (width 0.1524) (layer F.Cu) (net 3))
 (segment (start 185.706809 52.947278) (end 186.935 52.947278) (width 0.1524) (layer F.Cu) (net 3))
 (segment (start 187.127386 58.355456) (end 187.482842 58) (width 0.1524) (layer F.Cu) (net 6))
 (segment (start 187.6 58) (end 188.266897 57.333103) (width 0.3048) (layer F.Cu) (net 6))
 (segment (start 187.482842 58) (end 187.6 58) (width 0.3048) (layer F.Cu) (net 6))
 (segment (start 177.643153 57.229931) (end 178.440331 56.432753) (width 0.1524) (layer F.Cu) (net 12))
 (segment (start 177.643153 57.543153) (end 177.643153 57.229931) (width 0.1524) (layer F.Cu) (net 12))
 (segment (start 181.187691 59.133275) (end 181.133275 59.133275) (width 0.1524) (layer F.Cu) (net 13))
 (segment (start 181.541243 59.486827) (end 181.187691 59.133275) (width 0.1524) (layer F.Cu) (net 13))
 (segment (start 181.133275 59.133275) (end 180.9 58.9) (width 0.1524) (layer F.Cu) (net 13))
 (segment (start 180.9 58.9) (end 179.9 58.9) (width 0.1524) (layer F.Cu) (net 13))
 (segment (start 179.9 58.9) (end 179.6 59.2) (width 0.1524) (layer F.Cu) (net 13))
 (segment (start 179.3 59.2) (end 178.756847 58.656847) (width 0.1524) (layer F.Cu) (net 13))
 (segment (start 179.6 59.2) (end 179.3 59.2) (width 0.1524) (layer F.Cu) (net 13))
 (segment (start 179.132753 57.118647) (end 179.857053 57.842947) (width 0.1524) (layer F.Cu) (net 9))
 (segment (start 179.126225 57.118647) (end 179.132753 57.118647) (width 0.1524) (layer F.Cu) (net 9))
 (segment (start 181.470534 58.850432) (end 181.824086 59.203984) (width 0.1524) (layer F.Cu) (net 9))
 (segment (start 180.760033 58.139931) (end 181.470534 58.850432) (width 0.1524) (layer F.Cu) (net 9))
 (segment (start 180.154037 58.139931) (end 180.760033 58.139931) (width 0.1524) (layer F.Cu) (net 9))
 (segment (start 179.857053 57.842947) (end 180.154037 58.139931) (width 0.1524) (layer F.Cu) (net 9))
 (segment (start 188 54.4) (end 188 53.985) (width 0.1524) (layer F.Cu) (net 10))
 (segment (start 186.995189 55.404811) (end 188 54.4) (width 0.1524) (layer F.Cu) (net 10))
 (segment (start 186.278858 57.506928) (end 186.995189 56.790597) (width 0.1524) (layer F.Cu) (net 10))
 (segment (start 186.995189 56.790597) (end 186.995189 55.404811) (width 0.1524) (layer F.Cu) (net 10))
 (segment (start 187.3 57.051472) (end 187.3 56.08) (width 0.1524) (layer F.Cu) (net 14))
 (segment (start 186.561701 57.789771) (end 187.3 57.051472) (width 0.1524) (layer F.Cu) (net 14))
 (segment (start 189 54.38) (end 189 53.985) (width 0.1524) (layer F.Cu) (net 14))
 (segment (start 187.3 56.08) (end 189 54.38) (width 0.1524) (layer F.Cu) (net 14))
 (segment (start 184.241809 53.982278) (end 184.306809 54.047278) (width 0.1524) (layer F.Cu) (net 2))
 (segment (start 182.974809 53.982278) (end 184.241809 53.982278) (width 0.1524) (layer F.Cu) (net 2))
 (segment (start 186.066725 56.587691) (end 186.066725 56.533275) (width 0.1524) (layer F.Cu) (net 2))
 (segment (start 185.713173 56.941243) (end 186.066725 56.587691) (width 0.1524) (layer F.Cu) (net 2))
 (segment (start 186.066725 56.533275) (end 186.2 56.4) (width 0.1524) (layer F.Cu) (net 2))
 (segment (start 186.2 56.4) (end 186.2 56) (width 0.1524) (layer F.Cu) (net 2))
 (segment (start 186.2 56) (end 185.7 55.5) (width 0.1524) (layer F.Cu) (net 2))
 (segment (start 185.7 55.5) (end 184.9 55.5) (width 0.1524) (layer F.Cu) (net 2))
 (segment (start 184.306809 54.906809) (end 184.306809 54.047278) (width 0.1524) (layer F.Cu) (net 2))
 (segment (start 184.9 55.5) (end 184.306809 54.906809) (width 0.1524) (layer F.Cu) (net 2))
 (segment (start 193 55.3) (end 193 53.3) (width 0.3048) (layer F.Cu) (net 5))
 (segment (start 192.7 55.6) (end 193 55.3) (width 0.3048) (layer F.Cu) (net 5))
 (segment (start 189.133103 56.466897) (end 190 55.6) (width 0.3048) (layer F.Cu) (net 5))
 (segment (start 190 55.6) (end 192.7 55.6) (width 0.3048) (layer F.Cu) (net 5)))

